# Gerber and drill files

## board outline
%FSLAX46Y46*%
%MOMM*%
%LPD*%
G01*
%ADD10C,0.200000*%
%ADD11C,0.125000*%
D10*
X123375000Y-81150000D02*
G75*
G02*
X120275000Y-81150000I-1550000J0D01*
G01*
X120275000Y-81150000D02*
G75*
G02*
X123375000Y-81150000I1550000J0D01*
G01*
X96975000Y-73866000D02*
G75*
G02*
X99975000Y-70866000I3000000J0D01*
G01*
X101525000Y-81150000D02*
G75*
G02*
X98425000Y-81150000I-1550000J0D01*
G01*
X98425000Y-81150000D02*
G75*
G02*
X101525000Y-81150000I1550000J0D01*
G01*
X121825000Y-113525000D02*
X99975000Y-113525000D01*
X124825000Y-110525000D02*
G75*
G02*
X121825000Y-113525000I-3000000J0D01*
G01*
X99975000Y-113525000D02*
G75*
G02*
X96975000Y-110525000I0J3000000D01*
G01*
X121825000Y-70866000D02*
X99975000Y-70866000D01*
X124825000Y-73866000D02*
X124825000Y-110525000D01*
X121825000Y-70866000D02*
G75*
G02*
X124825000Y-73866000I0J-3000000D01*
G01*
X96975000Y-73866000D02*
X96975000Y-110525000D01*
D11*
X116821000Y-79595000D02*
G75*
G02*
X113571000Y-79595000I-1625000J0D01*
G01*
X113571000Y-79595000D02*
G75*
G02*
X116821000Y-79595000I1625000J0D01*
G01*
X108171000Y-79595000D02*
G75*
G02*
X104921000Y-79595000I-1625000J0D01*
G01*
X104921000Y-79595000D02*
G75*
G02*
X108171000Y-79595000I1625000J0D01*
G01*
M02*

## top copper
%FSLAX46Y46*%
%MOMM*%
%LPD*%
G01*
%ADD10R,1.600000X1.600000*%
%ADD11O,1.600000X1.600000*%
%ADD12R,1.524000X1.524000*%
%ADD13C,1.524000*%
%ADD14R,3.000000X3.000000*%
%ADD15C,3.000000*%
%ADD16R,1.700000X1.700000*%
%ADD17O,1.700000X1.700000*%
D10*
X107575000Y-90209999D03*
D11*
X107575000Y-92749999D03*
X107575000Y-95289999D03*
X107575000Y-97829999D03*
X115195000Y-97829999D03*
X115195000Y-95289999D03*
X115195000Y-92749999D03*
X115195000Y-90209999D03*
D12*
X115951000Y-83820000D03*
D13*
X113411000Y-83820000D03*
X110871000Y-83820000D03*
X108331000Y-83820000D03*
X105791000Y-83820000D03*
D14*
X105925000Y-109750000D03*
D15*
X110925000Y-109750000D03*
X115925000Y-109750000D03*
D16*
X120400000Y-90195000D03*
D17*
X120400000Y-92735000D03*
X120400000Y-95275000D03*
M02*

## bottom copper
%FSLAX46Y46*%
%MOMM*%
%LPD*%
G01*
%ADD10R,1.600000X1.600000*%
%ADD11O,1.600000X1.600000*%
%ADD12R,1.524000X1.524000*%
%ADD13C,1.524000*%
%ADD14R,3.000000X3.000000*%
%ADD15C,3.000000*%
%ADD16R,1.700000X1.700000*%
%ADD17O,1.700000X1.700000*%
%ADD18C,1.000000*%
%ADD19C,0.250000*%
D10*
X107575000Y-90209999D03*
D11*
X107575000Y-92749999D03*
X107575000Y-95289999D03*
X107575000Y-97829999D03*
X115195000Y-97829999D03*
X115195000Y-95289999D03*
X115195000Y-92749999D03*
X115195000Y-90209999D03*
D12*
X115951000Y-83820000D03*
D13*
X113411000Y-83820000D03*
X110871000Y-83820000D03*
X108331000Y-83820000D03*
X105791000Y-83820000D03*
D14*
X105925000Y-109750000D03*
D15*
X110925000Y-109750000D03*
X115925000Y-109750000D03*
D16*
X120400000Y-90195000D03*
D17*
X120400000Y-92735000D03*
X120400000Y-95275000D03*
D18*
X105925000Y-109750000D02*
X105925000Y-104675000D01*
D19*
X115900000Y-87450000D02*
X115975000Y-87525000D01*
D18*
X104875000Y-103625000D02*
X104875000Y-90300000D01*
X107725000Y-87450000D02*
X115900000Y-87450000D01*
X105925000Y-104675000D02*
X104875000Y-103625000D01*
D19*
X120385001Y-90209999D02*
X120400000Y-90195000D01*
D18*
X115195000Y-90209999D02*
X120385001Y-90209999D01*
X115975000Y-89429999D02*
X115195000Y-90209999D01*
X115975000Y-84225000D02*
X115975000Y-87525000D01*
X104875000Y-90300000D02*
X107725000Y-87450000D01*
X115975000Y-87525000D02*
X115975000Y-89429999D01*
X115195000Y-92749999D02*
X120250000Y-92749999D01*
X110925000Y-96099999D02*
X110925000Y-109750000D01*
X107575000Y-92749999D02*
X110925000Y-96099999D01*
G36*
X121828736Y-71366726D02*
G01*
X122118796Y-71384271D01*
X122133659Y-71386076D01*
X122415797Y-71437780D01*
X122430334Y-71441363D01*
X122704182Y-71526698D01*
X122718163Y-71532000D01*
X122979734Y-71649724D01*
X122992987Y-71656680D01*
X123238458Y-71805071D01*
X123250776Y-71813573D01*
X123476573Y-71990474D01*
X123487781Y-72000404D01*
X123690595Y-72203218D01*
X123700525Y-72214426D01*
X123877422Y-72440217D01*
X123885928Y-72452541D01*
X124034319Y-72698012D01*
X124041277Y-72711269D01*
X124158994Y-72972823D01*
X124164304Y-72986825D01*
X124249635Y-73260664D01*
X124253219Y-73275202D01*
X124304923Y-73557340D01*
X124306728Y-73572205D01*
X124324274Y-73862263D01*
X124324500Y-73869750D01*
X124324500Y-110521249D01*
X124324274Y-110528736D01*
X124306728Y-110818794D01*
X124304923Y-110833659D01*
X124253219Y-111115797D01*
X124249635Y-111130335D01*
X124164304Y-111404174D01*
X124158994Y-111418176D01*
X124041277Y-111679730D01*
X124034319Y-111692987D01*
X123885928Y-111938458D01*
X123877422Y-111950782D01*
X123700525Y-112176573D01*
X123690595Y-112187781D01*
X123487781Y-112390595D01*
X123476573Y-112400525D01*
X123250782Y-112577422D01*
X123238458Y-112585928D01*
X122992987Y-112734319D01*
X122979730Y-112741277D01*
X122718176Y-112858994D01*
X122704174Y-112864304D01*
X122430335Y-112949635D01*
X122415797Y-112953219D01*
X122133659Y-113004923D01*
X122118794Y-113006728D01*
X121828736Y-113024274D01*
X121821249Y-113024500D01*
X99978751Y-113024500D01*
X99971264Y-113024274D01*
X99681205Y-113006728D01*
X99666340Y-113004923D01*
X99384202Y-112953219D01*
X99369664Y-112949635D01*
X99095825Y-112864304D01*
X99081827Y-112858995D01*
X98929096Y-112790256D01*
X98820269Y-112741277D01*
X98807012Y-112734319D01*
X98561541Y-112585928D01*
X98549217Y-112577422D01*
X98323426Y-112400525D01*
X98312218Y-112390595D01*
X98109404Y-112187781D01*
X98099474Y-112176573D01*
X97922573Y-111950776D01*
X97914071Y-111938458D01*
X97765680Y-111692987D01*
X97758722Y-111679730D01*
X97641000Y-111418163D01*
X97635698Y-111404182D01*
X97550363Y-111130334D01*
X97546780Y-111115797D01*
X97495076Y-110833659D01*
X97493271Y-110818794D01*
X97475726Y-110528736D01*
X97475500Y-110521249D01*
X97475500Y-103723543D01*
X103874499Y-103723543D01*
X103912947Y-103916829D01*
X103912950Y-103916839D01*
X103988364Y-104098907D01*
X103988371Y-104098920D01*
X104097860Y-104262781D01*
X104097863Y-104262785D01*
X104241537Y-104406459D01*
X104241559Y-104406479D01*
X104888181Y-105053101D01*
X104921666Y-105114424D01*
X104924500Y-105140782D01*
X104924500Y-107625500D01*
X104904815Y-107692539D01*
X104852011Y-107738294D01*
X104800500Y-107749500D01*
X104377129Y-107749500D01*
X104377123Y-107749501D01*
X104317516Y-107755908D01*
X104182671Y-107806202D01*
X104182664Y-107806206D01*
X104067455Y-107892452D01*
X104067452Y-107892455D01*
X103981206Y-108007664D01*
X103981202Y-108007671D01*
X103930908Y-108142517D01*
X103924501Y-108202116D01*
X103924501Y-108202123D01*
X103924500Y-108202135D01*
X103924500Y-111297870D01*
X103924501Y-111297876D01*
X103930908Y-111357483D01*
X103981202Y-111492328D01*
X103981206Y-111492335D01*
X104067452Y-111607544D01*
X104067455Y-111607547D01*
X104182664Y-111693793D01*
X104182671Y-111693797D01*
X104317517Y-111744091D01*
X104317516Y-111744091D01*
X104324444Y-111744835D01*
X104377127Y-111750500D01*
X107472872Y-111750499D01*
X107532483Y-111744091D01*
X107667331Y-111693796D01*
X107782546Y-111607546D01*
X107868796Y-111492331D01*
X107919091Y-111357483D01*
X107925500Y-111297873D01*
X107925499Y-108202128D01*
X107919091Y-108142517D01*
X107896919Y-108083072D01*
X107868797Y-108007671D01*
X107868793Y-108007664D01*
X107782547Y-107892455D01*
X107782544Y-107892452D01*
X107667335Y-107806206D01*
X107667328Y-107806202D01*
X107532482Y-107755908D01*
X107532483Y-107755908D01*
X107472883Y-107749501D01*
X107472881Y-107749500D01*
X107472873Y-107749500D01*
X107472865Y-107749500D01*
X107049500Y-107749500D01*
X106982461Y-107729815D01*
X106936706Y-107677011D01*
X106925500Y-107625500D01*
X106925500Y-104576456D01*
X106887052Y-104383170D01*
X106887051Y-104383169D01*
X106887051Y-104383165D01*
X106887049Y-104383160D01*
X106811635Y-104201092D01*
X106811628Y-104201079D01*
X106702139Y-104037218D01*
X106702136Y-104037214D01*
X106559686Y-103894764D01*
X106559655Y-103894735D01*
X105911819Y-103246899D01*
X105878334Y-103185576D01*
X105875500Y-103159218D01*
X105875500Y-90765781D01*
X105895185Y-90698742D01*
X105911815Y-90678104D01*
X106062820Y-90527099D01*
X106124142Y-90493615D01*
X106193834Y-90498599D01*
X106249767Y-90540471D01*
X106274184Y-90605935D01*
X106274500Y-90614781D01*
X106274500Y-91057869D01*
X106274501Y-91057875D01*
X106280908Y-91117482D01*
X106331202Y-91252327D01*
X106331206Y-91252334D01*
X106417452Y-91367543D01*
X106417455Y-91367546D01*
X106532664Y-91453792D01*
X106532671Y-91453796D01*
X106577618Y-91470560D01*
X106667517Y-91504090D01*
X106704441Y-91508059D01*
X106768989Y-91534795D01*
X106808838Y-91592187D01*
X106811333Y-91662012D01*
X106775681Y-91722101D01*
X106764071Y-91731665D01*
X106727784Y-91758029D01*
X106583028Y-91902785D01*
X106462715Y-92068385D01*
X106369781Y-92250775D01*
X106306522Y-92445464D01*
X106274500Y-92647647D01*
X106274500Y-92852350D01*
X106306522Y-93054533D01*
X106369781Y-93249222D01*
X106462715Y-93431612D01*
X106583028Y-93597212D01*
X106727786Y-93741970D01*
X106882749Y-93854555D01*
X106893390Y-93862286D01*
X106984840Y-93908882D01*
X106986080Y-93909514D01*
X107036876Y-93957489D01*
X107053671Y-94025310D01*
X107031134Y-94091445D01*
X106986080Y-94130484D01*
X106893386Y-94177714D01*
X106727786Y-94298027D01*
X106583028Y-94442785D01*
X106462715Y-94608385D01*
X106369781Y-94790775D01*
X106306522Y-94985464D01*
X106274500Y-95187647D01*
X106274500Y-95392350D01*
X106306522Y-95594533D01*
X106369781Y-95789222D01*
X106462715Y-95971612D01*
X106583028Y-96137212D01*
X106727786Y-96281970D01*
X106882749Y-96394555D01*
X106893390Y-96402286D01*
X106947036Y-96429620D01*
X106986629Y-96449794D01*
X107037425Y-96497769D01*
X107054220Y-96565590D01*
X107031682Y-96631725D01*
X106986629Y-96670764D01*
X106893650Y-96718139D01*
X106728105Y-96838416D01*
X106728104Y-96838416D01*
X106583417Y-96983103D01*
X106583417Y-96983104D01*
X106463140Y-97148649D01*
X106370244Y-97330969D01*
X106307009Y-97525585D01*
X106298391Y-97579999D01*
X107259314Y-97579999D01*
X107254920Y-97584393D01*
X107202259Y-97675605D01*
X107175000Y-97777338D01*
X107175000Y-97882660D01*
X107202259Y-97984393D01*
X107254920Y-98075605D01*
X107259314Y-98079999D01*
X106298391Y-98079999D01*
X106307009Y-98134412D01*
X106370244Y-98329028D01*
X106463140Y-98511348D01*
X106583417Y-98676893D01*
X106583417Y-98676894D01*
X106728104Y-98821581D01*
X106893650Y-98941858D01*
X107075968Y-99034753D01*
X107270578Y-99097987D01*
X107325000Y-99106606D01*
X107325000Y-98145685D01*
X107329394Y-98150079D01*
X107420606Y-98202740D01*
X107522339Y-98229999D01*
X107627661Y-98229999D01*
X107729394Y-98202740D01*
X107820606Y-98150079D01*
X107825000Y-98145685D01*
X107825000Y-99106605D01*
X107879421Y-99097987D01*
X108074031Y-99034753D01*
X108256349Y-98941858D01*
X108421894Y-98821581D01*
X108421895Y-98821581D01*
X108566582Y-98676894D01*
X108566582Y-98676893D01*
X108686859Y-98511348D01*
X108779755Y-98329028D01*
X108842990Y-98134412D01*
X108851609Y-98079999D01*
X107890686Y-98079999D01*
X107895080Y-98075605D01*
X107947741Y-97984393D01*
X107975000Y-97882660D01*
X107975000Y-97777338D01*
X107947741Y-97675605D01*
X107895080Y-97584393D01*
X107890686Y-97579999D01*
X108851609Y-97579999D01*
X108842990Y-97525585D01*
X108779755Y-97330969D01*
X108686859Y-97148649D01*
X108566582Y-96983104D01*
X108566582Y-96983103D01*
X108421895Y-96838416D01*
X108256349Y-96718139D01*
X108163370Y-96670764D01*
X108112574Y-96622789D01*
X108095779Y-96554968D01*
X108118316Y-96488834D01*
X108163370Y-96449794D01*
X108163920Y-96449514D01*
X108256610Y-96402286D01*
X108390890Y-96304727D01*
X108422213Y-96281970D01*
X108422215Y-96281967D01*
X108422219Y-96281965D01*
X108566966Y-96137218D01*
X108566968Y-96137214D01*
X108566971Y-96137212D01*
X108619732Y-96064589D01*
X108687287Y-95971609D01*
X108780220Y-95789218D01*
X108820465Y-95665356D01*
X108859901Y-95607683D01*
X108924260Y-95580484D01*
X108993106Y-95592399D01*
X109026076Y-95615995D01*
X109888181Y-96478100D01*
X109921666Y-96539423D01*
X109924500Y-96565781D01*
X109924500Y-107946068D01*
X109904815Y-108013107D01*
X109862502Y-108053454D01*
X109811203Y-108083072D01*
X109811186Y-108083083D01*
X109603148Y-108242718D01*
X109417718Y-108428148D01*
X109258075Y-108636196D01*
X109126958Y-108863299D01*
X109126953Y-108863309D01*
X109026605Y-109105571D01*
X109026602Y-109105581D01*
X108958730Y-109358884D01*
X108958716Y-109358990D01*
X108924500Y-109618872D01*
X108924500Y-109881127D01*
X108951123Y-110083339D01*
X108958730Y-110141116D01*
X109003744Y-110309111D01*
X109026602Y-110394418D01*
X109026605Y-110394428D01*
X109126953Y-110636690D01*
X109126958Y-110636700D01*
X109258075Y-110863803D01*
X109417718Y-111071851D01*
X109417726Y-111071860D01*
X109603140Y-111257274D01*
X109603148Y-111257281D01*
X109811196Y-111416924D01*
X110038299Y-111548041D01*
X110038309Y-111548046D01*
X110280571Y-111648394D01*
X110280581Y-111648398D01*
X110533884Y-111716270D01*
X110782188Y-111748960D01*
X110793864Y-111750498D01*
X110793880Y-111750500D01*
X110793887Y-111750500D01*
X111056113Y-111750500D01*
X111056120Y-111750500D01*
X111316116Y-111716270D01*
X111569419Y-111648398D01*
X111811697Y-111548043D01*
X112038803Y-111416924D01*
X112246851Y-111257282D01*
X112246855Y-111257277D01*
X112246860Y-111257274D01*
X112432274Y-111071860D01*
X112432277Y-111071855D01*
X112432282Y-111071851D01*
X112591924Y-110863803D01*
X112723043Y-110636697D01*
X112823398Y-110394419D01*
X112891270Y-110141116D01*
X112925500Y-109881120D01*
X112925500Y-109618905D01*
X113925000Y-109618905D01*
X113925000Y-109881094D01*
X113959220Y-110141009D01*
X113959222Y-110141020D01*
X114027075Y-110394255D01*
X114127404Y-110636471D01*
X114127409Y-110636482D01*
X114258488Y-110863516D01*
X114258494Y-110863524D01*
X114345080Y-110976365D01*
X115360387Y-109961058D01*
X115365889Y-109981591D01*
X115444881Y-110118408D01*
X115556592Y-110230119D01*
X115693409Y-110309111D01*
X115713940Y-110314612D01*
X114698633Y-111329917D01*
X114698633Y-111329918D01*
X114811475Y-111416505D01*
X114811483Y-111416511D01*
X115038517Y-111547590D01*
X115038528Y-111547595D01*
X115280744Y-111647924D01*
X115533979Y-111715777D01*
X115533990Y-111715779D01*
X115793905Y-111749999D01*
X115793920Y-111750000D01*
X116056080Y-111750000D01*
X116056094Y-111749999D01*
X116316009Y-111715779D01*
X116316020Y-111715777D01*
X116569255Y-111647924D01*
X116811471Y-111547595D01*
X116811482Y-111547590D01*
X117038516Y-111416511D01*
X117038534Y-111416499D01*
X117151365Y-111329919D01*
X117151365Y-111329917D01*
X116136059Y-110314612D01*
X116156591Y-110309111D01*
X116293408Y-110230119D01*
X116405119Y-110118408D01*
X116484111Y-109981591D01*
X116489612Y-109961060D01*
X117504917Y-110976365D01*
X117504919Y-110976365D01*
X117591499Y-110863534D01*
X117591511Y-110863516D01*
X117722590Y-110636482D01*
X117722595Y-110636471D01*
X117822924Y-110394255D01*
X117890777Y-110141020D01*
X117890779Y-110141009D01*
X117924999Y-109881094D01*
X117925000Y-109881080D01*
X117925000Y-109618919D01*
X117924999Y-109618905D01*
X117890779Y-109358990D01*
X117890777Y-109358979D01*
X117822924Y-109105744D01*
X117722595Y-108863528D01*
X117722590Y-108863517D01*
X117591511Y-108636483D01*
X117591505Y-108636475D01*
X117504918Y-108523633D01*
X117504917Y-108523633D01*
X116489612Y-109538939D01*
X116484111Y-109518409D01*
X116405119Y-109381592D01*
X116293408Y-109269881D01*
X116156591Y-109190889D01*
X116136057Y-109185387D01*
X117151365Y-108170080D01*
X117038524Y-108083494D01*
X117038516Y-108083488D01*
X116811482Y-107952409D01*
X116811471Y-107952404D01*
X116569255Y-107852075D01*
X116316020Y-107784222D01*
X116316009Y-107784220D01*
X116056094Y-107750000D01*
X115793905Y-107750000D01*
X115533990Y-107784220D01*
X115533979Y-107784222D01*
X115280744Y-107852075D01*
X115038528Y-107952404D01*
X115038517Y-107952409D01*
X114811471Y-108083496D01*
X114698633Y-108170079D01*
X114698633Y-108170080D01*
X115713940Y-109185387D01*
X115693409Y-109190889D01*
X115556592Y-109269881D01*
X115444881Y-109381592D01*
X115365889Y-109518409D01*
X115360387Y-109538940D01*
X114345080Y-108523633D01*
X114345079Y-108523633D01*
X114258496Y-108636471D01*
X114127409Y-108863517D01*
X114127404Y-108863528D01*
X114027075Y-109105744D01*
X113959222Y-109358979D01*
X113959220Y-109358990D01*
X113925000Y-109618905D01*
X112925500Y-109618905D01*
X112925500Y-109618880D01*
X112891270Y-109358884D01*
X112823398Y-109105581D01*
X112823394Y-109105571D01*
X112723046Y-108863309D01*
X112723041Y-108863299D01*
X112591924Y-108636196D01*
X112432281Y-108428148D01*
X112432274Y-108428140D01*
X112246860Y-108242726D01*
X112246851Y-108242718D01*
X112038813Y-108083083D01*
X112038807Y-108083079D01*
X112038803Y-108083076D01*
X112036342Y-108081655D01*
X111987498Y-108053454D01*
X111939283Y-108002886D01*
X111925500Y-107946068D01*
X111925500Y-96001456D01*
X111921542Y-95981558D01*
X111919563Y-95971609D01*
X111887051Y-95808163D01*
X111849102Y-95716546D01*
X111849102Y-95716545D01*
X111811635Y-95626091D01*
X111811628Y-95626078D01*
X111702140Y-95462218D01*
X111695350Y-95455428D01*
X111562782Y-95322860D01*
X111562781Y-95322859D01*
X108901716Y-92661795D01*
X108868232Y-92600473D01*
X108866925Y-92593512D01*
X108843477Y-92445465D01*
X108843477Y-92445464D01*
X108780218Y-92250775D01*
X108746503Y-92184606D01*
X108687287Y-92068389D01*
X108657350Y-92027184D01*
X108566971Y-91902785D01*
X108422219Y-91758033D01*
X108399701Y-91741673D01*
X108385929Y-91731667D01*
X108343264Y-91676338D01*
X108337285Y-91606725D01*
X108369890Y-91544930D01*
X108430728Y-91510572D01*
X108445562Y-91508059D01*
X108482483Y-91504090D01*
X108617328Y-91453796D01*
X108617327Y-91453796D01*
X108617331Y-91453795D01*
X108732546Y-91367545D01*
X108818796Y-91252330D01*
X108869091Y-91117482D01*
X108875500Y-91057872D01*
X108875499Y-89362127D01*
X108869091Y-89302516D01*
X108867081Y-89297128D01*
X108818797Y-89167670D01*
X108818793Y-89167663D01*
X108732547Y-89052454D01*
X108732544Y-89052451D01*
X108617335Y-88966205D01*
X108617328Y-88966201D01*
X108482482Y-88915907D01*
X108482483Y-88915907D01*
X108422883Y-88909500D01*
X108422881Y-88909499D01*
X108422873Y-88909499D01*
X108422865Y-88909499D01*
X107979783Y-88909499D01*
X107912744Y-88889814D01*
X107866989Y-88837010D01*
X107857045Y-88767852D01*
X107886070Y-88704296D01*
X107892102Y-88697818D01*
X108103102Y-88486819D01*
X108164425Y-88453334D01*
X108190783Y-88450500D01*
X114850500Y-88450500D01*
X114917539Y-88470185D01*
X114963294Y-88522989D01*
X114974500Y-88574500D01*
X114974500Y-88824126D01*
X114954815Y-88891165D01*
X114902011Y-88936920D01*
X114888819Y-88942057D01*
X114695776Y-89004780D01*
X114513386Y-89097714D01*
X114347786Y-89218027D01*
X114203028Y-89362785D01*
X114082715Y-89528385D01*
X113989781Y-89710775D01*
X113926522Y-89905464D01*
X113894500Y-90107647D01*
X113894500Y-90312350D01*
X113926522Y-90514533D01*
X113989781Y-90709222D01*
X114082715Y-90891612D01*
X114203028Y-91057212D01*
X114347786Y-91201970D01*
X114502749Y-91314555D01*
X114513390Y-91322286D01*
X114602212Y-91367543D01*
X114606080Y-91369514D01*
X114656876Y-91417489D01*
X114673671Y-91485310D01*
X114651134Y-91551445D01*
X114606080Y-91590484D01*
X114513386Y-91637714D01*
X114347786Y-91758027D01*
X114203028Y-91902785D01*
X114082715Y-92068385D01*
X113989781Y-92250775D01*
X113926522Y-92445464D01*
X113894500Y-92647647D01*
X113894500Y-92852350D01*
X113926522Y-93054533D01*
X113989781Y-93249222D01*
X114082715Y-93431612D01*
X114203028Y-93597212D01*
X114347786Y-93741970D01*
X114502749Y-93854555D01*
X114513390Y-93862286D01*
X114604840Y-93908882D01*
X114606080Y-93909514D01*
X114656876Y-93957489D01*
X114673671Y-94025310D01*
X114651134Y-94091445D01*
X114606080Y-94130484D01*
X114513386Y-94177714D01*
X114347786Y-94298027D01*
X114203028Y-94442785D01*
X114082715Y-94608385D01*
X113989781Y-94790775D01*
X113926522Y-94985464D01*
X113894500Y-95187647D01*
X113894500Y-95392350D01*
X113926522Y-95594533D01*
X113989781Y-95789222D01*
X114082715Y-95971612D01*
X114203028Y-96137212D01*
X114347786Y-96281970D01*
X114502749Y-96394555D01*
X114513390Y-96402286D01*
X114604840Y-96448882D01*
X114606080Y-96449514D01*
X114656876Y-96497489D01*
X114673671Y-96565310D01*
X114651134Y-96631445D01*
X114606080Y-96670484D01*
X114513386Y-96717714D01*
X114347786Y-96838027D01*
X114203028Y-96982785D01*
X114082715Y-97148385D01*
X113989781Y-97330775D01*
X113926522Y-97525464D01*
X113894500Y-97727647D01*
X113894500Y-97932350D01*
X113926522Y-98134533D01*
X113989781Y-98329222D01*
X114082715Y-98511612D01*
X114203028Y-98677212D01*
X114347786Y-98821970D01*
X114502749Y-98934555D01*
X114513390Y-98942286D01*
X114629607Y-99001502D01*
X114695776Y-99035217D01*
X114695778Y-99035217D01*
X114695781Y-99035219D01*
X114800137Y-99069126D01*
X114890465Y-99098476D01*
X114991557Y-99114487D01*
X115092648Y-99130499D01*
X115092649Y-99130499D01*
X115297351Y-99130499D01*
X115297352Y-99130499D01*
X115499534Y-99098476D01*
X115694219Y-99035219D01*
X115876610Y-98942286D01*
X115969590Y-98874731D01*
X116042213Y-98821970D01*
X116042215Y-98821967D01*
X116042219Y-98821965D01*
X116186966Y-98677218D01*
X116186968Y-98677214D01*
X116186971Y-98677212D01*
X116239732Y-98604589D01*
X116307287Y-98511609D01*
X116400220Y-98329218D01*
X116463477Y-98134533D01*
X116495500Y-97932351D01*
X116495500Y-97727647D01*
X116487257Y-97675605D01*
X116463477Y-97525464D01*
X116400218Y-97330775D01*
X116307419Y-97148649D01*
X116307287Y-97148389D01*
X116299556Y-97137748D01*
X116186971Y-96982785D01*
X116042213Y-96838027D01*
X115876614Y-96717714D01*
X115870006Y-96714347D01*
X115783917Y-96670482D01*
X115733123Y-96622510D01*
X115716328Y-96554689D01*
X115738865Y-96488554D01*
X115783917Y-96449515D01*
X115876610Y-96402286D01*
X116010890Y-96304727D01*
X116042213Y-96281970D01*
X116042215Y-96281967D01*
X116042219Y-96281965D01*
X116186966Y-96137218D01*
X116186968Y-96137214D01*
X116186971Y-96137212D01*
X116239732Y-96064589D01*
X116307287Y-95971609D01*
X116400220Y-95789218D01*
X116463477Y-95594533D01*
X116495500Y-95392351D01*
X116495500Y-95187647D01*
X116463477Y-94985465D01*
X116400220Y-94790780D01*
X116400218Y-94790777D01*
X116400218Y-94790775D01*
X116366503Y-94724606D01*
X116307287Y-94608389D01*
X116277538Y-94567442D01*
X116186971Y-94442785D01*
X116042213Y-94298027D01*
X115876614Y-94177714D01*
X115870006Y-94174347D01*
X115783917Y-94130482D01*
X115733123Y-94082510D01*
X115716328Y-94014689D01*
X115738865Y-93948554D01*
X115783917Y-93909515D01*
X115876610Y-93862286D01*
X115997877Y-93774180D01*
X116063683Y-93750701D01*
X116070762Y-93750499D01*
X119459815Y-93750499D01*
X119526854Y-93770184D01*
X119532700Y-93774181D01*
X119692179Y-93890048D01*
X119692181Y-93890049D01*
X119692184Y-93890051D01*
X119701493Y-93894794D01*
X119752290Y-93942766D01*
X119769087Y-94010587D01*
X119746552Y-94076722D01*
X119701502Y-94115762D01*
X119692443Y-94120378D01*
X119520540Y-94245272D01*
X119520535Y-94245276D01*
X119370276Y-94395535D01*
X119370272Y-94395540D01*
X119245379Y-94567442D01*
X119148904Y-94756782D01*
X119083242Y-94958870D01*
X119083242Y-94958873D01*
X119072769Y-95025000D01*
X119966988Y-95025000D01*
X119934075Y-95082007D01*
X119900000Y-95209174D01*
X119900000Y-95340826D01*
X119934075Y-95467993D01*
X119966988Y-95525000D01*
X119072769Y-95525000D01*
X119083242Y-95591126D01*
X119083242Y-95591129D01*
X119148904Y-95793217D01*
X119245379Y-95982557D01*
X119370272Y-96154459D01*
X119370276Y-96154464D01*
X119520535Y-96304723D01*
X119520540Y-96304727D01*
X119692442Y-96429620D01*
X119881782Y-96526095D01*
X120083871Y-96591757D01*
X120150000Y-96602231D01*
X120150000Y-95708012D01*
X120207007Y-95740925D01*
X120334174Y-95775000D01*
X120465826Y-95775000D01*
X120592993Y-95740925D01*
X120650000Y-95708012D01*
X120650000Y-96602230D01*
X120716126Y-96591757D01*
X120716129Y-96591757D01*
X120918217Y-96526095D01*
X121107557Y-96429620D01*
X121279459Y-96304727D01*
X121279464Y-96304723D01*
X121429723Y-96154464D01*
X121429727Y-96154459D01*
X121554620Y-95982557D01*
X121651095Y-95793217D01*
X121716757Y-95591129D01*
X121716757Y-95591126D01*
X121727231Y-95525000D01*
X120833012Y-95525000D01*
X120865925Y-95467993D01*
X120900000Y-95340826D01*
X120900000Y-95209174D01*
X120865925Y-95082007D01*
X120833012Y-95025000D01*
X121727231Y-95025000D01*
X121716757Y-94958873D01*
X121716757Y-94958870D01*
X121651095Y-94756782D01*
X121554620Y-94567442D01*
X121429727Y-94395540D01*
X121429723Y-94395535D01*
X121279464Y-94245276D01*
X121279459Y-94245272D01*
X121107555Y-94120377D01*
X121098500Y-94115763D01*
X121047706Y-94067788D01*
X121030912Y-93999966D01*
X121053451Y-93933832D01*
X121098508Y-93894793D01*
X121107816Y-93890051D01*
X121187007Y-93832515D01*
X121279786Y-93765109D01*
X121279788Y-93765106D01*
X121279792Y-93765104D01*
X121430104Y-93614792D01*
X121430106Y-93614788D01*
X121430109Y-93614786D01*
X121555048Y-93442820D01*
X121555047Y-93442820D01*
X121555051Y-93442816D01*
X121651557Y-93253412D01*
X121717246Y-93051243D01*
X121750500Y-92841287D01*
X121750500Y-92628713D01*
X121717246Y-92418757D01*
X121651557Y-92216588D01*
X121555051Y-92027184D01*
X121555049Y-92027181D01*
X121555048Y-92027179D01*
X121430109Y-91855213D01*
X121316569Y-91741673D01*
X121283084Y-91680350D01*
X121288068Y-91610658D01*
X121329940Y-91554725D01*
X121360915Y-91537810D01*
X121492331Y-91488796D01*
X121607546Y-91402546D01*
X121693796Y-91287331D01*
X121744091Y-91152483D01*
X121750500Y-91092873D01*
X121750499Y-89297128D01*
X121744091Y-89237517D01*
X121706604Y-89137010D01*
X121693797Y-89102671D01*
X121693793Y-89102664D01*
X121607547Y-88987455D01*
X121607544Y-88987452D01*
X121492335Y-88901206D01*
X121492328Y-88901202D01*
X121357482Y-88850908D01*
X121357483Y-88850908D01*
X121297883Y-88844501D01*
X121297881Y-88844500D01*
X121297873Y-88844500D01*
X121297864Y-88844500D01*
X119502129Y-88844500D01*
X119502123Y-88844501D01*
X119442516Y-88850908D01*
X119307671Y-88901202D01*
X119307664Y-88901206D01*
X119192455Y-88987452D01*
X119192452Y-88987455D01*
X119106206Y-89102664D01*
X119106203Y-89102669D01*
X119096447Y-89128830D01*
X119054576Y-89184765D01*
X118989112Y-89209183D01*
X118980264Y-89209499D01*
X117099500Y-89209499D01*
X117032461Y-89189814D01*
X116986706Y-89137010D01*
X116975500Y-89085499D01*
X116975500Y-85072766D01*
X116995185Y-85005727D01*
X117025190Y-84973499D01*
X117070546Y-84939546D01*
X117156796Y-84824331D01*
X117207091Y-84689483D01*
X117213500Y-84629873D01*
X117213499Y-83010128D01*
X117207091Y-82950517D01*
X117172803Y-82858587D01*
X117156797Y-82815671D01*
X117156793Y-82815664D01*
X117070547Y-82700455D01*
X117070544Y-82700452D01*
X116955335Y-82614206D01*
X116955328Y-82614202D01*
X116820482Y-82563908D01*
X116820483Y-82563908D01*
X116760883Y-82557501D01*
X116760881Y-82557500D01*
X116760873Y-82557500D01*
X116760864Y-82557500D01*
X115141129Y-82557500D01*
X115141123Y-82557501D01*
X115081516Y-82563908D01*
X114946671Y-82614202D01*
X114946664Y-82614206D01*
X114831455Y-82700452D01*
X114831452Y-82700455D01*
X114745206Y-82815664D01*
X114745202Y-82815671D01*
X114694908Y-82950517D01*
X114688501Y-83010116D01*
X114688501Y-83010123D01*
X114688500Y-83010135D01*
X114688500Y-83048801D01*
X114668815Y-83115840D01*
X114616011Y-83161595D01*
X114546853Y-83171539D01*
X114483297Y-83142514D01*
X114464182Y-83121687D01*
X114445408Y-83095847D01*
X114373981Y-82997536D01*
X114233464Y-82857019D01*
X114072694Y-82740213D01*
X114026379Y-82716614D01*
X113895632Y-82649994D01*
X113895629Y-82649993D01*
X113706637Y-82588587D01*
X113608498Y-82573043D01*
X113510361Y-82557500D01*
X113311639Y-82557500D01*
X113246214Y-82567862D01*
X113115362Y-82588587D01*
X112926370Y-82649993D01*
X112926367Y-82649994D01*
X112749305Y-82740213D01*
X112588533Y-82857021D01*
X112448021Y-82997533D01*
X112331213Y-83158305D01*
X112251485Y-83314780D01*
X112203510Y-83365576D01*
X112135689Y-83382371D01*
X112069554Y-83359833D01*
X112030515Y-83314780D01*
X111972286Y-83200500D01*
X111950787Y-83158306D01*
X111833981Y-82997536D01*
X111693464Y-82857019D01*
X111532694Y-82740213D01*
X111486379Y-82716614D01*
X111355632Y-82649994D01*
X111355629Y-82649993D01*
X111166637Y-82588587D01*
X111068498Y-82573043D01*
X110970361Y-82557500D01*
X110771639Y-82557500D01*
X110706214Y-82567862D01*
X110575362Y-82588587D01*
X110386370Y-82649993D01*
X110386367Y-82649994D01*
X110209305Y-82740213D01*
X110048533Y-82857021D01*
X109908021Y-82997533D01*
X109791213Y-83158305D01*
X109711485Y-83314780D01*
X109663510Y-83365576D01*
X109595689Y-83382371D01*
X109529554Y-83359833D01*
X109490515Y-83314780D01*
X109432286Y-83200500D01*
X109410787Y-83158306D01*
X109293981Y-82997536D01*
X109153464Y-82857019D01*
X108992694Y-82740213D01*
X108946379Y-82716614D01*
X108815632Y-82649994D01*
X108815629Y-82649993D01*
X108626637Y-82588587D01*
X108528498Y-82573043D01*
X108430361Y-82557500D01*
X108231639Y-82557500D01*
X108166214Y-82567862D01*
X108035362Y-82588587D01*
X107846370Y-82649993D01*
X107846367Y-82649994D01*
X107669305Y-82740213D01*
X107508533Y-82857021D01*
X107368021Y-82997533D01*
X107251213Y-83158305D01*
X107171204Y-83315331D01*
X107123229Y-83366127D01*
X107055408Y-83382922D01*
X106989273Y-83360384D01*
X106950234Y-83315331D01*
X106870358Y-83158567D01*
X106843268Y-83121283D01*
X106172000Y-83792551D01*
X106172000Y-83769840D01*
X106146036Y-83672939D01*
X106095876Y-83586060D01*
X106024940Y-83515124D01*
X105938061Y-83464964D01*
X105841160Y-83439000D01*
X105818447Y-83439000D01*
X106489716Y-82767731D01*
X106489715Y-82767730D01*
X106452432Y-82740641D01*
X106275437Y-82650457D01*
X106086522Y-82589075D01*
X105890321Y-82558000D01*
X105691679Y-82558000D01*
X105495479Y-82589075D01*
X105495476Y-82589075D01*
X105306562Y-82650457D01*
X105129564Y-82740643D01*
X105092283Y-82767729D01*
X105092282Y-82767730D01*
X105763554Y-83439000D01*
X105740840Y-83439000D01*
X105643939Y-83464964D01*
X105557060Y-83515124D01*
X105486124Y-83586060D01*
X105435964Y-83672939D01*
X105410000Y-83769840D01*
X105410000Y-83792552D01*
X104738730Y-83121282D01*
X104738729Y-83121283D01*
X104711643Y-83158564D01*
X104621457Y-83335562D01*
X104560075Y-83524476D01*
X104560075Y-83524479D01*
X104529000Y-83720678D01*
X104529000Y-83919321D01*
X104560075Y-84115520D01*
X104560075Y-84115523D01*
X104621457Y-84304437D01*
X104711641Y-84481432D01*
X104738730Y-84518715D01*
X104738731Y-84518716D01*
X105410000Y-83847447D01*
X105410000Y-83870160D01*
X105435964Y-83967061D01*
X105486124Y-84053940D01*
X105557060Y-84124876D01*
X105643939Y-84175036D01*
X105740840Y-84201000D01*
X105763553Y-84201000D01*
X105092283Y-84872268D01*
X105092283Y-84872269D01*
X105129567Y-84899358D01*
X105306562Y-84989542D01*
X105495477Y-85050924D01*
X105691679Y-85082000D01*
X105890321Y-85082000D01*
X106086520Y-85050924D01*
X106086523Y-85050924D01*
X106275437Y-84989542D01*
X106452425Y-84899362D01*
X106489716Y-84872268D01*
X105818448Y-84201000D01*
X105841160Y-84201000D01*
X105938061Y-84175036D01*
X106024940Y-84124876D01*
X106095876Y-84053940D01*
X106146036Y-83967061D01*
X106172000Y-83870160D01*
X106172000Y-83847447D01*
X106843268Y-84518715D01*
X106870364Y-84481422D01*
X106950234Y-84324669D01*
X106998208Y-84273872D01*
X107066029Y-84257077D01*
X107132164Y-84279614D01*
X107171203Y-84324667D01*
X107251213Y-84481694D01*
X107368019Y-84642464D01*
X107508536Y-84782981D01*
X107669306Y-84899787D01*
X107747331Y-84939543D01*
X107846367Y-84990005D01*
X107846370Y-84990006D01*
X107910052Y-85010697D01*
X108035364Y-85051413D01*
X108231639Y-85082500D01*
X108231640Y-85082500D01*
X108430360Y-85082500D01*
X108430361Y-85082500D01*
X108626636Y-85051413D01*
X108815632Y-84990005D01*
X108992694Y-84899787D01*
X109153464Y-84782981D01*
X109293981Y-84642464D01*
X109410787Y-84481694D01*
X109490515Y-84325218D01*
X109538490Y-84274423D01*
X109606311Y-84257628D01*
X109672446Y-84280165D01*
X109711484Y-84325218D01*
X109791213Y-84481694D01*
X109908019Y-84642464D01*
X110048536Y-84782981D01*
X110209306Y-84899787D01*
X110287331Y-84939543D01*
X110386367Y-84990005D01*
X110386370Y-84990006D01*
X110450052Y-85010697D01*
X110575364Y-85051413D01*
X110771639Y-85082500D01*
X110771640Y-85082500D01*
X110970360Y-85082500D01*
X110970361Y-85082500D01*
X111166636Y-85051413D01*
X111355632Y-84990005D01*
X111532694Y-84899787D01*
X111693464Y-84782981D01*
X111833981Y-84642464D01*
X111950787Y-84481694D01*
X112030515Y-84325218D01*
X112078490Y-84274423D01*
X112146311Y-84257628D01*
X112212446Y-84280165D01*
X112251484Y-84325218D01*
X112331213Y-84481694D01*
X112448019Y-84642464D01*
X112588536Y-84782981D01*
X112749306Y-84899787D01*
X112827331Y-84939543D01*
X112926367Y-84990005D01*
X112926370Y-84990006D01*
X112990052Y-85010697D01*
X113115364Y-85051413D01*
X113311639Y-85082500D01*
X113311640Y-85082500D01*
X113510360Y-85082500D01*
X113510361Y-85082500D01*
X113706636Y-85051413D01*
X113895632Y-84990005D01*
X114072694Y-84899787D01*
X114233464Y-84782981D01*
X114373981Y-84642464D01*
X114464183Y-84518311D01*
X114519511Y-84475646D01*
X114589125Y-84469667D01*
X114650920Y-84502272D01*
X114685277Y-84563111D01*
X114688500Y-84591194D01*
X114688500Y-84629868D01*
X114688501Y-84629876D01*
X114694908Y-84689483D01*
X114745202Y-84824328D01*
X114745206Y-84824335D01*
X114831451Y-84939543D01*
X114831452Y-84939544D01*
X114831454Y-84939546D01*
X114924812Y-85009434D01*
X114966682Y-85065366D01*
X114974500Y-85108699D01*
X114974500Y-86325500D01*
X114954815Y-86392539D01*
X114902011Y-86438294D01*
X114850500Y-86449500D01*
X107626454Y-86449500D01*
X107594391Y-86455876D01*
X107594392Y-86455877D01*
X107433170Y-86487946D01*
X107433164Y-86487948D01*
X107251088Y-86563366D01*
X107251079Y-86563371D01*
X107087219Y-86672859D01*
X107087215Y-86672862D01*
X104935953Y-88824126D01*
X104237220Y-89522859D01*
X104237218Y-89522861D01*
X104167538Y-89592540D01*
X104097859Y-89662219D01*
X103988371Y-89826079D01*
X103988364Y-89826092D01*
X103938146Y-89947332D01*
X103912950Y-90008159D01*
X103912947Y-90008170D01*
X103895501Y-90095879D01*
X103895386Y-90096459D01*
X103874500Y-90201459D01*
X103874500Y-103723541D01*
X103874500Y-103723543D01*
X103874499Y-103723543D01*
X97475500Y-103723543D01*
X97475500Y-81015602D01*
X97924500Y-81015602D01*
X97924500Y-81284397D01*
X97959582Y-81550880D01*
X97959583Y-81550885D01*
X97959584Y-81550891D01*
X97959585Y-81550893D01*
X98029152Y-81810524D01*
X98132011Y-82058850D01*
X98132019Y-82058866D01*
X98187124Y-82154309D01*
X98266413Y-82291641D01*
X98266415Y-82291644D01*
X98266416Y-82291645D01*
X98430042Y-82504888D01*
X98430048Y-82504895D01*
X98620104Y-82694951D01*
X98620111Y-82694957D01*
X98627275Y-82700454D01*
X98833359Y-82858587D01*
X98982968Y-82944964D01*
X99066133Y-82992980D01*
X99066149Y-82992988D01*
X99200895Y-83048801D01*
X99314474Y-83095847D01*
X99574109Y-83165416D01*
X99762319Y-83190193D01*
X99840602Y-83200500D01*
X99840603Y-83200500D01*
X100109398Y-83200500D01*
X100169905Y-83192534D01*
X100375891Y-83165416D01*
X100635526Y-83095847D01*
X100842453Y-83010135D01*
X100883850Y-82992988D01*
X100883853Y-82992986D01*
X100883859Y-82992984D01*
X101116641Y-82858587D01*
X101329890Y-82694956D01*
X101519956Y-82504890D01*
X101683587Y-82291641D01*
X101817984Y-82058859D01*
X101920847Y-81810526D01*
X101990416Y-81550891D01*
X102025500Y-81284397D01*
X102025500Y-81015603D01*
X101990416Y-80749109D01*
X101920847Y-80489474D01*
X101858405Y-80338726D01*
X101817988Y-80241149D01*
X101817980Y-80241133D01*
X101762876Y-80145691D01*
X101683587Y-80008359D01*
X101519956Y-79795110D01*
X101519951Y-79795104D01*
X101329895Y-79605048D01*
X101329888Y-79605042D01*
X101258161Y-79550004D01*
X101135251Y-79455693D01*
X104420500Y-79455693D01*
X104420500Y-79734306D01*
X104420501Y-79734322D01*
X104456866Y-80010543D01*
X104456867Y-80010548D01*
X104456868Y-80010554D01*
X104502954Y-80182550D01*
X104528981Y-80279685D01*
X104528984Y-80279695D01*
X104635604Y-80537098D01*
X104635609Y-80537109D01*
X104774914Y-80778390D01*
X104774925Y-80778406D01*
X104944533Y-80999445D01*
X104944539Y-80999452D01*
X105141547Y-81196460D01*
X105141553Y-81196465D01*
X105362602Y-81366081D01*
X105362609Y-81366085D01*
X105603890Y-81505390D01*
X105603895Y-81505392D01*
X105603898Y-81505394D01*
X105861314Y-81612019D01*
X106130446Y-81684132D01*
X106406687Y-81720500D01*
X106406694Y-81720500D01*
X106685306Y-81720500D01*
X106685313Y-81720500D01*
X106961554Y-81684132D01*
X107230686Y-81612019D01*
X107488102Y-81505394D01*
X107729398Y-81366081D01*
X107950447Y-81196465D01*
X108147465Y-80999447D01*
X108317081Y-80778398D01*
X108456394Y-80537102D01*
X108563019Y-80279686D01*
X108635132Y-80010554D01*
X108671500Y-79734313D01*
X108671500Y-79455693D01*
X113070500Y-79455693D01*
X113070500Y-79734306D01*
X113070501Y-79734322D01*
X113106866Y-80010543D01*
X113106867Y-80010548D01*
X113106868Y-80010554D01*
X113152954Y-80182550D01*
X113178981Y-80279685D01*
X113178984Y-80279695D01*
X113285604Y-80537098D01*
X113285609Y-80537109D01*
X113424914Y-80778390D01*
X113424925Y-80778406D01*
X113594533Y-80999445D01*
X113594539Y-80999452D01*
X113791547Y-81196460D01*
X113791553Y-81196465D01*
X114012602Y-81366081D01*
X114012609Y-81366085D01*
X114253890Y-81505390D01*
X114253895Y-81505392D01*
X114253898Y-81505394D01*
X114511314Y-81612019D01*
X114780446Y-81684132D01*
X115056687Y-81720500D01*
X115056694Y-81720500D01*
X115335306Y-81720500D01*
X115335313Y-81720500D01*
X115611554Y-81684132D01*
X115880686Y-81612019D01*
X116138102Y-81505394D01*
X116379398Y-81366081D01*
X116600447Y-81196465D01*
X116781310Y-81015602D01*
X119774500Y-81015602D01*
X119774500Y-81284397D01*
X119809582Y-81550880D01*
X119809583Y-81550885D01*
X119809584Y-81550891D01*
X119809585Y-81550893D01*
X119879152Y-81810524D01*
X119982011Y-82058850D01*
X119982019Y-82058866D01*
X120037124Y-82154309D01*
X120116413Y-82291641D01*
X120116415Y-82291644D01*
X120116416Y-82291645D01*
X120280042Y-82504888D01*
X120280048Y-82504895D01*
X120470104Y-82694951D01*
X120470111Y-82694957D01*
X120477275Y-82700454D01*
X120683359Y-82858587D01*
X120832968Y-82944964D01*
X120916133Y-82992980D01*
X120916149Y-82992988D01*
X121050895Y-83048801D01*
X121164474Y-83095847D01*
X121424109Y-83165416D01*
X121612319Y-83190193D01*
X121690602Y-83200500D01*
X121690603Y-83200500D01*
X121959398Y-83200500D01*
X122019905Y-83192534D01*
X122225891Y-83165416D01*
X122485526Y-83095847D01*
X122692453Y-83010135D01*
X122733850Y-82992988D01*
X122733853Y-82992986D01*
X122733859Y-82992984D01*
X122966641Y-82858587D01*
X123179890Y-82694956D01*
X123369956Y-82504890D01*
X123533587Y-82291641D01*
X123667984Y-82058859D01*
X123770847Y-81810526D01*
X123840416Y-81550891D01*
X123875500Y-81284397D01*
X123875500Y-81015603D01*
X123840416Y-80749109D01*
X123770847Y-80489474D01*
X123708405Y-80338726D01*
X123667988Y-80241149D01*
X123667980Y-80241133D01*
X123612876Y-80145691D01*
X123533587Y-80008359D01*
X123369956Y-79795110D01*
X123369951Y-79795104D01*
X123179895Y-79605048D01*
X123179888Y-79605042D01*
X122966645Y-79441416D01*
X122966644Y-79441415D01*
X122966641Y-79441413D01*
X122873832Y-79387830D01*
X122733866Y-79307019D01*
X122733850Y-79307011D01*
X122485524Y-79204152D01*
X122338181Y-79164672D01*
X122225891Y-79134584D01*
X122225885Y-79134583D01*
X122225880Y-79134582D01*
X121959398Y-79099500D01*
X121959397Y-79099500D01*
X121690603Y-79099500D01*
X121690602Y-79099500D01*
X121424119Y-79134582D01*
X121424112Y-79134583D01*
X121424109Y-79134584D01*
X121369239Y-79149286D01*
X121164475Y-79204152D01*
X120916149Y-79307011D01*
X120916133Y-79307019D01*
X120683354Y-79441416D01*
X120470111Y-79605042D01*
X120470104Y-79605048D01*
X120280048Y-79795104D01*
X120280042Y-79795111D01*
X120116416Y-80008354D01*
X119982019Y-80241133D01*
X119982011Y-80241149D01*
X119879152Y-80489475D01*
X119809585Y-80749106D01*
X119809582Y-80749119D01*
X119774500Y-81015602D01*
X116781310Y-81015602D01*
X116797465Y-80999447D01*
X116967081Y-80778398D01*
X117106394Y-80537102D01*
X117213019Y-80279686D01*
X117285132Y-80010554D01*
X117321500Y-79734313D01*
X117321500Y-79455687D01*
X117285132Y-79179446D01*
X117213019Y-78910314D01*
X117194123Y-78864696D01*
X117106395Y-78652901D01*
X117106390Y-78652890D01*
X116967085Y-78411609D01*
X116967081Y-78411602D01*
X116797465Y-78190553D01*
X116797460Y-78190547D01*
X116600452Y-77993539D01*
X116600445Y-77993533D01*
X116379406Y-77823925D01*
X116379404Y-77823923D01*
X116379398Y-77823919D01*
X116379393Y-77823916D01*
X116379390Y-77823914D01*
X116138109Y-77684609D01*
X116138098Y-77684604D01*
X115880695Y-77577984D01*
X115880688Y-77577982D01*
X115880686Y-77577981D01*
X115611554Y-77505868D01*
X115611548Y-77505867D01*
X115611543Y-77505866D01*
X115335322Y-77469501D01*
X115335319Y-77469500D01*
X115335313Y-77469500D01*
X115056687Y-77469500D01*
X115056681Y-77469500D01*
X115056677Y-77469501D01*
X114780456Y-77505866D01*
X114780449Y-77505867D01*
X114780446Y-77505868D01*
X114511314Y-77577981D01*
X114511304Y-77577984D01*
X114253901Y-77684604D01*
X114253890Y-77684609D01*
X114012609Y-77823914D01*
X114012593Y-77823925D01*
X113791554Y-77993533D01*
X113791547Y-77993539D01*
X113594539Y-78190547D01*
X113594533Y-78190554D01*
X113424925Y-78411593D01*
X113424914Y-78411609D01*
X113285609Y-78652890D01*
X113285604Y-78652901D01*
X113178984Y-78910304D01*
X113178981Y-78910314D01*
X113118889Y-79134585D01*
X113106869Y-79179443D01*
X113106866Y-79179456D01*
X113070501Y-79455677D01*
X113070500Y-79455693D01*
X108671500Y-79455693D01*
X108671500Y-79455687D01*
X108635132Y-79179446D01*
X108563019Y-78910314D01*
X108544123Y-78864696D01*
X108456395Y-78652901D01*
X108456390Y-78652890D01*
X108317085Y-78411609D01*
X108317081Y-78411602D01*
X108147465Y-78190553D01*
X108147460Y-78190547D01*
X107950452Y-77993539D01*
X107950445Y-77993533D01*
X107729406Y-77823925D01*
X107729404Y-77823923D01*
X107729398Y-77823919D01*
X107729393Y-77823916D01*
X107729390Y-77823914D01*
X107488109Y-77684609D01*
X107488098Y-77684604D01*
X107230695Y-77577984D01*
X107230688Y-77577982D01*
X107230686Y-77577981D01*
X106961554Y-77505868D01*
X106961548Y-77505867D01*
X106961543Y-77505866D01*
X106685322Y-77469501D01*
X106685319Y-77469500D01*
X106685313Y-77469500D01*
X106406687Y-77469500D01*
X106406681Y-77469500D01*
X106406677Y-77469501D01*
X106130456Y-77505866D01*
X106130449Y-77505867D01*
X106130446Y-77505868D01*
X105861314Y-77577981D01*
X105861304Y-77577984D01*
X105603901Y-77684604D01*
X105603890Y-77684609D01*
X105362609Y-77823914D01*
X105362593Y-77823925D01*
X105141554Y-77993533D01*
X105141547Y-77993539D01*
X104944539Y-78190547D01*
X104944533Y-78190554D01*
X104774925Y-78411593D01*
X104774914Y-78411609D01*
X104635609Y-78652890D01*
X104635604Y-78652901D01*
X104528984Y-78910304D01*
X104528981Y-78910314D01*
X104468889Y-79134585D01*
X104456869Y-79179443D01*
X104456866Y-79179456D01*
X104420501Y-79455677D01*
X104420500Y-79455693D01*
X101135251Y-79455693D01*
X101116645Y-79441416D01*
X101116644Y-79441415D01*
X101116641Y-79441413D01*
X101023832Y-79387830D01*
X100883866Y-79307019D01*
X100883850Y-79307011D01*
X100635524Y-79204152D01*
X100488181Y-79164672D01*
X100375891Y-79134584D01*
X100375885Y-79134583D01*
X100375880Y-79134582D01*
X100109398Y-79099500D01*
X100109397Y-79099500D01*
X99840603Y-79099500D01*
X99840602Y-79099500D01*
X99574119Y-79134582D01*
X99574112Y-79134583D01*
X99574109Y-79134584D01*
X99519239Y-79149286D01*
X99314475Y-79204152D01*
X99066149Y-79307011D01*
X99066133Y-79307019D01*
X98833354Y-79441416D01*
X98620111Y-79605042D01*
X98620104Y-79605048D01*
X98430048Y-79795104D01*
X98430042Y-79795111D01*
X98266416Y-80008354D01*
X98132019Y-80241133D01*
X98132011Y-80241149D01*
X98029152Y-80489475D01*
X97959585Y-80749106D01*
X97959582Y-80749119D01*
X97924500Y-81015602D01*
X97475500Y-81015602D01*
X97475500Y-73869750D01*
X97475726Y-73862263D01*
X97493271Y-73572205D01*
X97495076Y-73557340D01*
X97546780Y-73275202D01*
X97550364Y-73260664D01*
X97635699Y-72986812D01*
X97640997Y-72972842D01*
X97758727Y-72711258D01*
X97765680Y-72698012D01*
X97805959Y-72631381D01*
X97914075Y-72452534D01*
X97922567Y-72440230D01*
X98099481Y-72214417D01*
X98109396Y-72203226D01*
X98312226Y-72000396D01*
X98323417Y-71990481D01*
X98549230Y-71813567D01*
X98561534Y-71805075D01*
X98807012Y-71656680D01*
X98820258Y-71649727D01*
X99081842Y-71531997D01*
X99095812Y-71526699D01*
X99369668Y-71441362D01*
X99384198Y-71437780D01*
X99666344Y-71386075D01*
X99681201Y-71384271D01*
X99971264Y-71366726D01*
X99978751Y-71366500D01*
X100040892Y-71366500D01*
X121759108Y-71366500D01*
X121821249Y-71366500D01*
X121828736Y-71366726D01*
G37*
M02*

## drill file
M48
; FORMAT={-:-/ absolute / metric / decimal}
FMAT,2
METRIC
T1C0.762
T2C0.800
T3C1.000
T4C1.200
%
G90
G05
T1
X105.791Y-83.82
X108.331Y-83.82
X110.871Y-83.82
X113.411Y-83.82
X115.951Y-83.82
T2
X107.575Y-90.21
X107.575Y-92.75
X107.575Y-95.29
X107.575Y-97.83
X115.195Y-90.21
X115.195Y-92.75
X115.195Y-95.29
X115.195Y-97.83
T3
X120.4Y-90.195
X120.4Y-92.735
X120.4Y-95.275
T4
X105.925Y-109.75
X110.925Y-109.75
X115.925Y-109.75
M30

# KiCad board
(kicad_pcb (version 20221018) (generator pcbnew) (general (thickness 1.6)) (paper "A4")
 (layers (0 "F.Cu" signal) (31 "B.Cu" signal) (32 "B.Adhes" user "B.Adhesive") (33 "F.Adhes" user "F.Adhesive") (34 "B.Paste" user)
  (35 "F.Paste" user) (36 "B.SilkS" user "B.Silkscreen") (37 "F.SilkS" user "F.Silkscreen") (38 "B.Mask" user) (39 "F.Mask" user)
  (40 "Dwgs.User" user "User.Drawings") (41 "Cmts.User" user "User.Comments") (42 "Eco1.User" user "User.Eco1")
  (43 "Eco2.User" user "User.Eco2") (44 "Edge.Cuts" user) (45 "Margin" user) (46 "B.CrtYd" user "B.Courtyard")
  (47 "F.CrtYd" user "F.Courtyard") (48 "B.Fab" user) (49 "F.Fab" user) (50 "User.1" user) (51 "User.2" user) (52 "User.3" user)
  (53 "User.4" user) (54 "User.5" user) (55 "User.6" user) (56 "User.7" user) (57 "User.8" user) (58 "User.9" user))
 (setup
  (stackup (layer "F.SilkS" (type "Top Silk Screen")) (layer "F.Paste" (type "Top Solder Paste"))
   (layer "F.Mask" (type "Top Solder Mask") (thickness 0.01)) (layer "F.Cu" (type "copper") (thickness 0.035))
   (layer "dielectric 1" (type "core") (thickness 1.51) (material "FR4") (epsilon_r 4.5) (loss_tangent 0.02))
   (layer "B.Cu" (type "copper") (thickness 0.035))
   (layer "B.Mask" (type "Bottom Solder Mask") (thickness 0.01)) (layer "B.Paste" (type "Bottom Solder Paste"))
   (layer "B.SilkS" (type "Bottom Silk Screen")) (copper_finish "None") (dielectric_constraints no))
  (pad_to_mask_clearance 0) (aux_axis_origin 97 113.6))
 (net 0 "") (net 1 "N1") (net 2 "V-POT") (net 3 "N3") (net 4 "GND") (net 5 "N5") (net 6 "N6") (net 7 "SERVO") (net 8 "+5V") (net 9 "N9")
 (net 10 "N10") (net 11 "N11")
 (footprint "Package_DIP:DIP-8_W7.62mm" (layer "F.Cu") (at 107.575 90.209999)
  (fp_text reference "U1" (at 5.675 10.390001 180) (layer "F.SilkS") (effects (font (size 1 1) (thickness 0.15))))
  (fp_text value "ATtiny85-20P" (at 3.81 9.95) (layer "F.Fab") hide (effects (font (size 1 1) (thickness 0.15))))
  (pad "1" thru_hole rect (at 0 0) (size 1.6 1.6) (drill 0.8) (layers "*.Cu" "*.Mask") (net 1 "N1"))
  (pad "2" thru_hole oval (at 0 2.54) (size 1.6 1.6) (drill 0.8) (layers "*.Cu" "*.Mask") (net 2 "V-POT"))
  (pad "3" thru_hole oval (at 0 5.08) (size 1.6 1.6) (drill 0.8) (layers "*.Cu" "*.Mask") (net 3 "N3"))
  (pad "4" thru_hole oval (at 0 7.62) (size 1.6 1.6) (drill 0.8) (layers "*.Cu" "*.Mask") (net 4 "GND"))
  (pad "5" thru_hole oval (at 7.62 7.62) (size 1.6 1.6) (drill 0.8) (layers "*.Cu" "*.Mask") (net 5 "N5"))
  (pad "6" thru_hole oval (at 7.62 5.08) (size 1.6 1.6) (drill 0.8) (layers "*.Cu" "*.Mask") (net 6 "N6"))
  (pad "7" thru_hole oval (at 7.62 2.54) (size 1.6 1.6) (drill 0.8) (layers "*.Cu" "*.Mask") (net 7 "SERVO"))
  (pad "8" thru_hole oval (at 7.62 0) (size 1.6 1.6) (drill 0.8) (layers "*.Cu" "*.Mask") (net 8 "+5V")))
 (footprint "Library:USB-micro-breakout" (layer "F.Cu") (at 110.871 83.82 180) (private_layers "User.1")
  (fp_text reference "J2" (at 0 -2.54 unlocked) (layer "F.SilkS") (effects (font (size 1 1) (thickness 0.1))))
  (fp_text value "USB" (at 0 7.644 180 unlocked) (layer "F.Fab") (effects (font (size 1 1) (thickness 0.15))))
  (fp_circle (center -4.325 4.225) (end -2.7 4.225) (stroke (width 0.125) (type default)) (fill none) (layer "Edge.Cuts"))
  (fp_circle (center 4.325 4.225) (end 5.95 4.225) (stroke (width 0.125) (type default)) (fill none) (layer "Edge.Cuts"))
  (pad "1" thru_hole rect (at -5.08 0 180) (size 1.524 1.524) (drill 0.762) (layers "*.Cu" "*.Mask") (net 8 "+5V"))
  (pad "2" thru_hole circle (at -2.54 0 180) (size 1.524 1.524) (drill 0.762) (layers "*.Cu" "*.Mask") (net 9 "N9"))
  (pad "3" thru_hole circle (at 0 0 180) (size 1.524 1.524) (drill 0.762) (layers "*.Cu" "*.Mask") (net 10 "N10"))
  (pad "4" thru_hole circle (at 2.54 0 180) (size 1.524 1.524) (drill 0.762) (layers "*.Cu" "*.Mask") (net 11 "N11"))
  (pad "5" thru_hole circle (at 5.08 0 180) (size 1.524 1.524) (drill 0.762) (layers "*.Cu" "*.Mask") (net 4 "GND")))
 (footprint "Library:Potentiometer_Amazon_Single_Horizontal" (layer "F.Cu") (at 105.925 109.75 90)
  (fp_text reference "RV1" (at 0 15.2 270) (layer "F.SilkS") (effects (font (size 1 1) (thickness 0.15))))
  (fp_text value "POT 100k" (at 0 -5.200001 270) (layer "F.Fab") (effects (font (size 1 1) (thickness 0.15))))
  (pad "1" thru_hole rect (at 0 0 270) (size 3 3) (drill 1.2) (layers "*.Cu" "*.Mask") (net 8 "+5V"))
  (pad "2" thru_hole circle (at 0 5 270) (size 3 3) (drill 1.2) (layers "*.Cu" "*.Mask") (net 2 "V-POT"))
  (pad "3" thru_hole circle (at 0 10 270) (size 3 3) (drill 1.2) (layers "*.Cu" "*.Mask") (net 4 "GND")))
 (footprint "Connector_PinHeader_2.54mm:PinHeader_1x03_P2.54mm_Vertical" (layer "F.Cu") (at 120.4 90.195)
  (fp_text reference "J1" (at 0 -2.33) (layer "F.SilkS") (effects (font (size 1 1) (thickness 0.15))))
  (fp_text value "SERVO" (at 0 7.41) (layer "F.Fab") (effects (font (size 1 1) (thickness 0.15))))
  (pad "1" thru_hole rect (at 0 0) (size 1.7 1.7) (drill 1) (layers "*.Cu" "*.Mask") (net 8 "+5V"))
  (pad "2" thru_hole oval (at 0 2.54) (size 1.7 1.7) (drill 1) (layers "*.Cu" "*.Mask") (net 7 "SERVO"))
  (pad "3" thru_hole oval (at 0 5.08) (size 1.7 1.7) (drill 1) (layers "*.Cu" "*.Mask") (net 4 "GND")))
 (gr_circle (center 121.825 81.15) (end 123.375 81.15) (stroke (width 0.2) (type solid)) (fill none) (layer "Edge.Cuts"))
 (gr_arc (start 96.975 73.866) (mid 97.85368 71.74468) (end 99.975 70.866) (stroke (width 0.2) (type solid)) (layer "Edge.Cuts"))
 (gr_circle (center 99.975 81.15) (end 101.525 81.15) (stroke (width 0.2) (type solid)) (fill none) (layer "Edge.Cuts"))
 (gr_line (start 121.825 113.525) (end 99.975 113.525) (stroke (width 0.2) (type solid)) (layer "Edge.Cuts"))
 (gr_arc (start 124.825 110.525) (mid 123.94632 112.64632) (end 121.825 113.525) (stroke (width 0.2) (type solid)) (layer "Edge.Cuts"))
 (gr_arc (start 99.975 113.525) (mid 97.85368 112.64632) (end 96.975 110.525) (stroke (width 0.2) (type solid)) (layer "Edge.Cuts"))
 (gr_line (start 121.825 70.866) (end 99.975 70.866) (stroke (width 0.2) (type solid)) (layer "Edge.Cuts"))
 (gr_line (start 124.825 73.866) (end 124.825 110.525) (stroke (width 0.2) (type solid)) (layer "Edge.Cuts"))
 (gr_arc (start 121.825 70.866) (mid 123.94632 71.74468) (end 124.825 73.866) (stroke (width 0.2) (type solid)) (layer "Edge.Cuts"))
 (gr_line (start 96.975 73.866) (end 96.975 110.525) (stroke (width 0.2) (type solid)) (layer "Edge.Cuts"))
 (segment (start 105.925 109.75) (end 105.925 104.675) (width 1) (layer "B.Cu") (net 8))
 (segment (start 115.9 87.45) (end 115.975 87.525) (width 0.25) (layer "B.Cu") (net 8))
 (segment (start 104.875 103.625) (end 104.875 90.3) (width 1) (layer "B.Cu") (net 8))
 (segment (start 107.725 87.45) (end 115.9 87.45) (width 1) (layer "B.Cu") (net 8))
 (segment (start 105.925 104.675) (end 104.875 103.625) (width 1) (layer "B.Cu") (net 8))
 (segment (start 120.385001 90.209999) (end 120.4 90.195) (width 0.25) (layer "B.Cu") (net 8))
 (segment (start 115.195 90.209999) (end 120.385001 90.209999) (width 1) (layer "B.Cu") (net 8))
 (segment (start 115.975 89.429999) (end 115.195 90.209999) (width 1) (layer "B.Cu") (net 8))
 (segment (start 115.975 84.225) (end 115.975 87.525) (width 1) (layer "B.Cu") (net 8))
 (segment (start 104.875 90.3) (end 107.725 87.45) (width 1) (layer "B.Cu") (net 8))
 (segment (start 115.975 87.525) (end 115.975 89.429999) (width 1) (layer "B.Cu") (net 8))
 (segment (start 115.195 92.749999) (end 120.25 92.749999) (width 1) (layer "B.Cu") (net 7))
 (segment (start 110.925 96.099999) (end 110.925 109.75) (width 1) (layer "B.Cu") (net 2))
 (segment (start 107.575 92.749999) (end 110.925 96.099999) (width 1) (layer "B.Cu") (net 2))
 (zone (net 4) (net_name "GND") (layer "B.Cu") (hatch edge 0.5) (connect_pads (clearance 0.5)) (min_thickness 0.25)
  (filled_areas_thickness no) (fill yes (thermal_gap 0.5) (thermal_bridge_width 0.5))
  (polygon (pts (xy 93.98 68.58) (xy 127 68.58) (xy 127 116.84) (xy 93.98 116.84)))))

